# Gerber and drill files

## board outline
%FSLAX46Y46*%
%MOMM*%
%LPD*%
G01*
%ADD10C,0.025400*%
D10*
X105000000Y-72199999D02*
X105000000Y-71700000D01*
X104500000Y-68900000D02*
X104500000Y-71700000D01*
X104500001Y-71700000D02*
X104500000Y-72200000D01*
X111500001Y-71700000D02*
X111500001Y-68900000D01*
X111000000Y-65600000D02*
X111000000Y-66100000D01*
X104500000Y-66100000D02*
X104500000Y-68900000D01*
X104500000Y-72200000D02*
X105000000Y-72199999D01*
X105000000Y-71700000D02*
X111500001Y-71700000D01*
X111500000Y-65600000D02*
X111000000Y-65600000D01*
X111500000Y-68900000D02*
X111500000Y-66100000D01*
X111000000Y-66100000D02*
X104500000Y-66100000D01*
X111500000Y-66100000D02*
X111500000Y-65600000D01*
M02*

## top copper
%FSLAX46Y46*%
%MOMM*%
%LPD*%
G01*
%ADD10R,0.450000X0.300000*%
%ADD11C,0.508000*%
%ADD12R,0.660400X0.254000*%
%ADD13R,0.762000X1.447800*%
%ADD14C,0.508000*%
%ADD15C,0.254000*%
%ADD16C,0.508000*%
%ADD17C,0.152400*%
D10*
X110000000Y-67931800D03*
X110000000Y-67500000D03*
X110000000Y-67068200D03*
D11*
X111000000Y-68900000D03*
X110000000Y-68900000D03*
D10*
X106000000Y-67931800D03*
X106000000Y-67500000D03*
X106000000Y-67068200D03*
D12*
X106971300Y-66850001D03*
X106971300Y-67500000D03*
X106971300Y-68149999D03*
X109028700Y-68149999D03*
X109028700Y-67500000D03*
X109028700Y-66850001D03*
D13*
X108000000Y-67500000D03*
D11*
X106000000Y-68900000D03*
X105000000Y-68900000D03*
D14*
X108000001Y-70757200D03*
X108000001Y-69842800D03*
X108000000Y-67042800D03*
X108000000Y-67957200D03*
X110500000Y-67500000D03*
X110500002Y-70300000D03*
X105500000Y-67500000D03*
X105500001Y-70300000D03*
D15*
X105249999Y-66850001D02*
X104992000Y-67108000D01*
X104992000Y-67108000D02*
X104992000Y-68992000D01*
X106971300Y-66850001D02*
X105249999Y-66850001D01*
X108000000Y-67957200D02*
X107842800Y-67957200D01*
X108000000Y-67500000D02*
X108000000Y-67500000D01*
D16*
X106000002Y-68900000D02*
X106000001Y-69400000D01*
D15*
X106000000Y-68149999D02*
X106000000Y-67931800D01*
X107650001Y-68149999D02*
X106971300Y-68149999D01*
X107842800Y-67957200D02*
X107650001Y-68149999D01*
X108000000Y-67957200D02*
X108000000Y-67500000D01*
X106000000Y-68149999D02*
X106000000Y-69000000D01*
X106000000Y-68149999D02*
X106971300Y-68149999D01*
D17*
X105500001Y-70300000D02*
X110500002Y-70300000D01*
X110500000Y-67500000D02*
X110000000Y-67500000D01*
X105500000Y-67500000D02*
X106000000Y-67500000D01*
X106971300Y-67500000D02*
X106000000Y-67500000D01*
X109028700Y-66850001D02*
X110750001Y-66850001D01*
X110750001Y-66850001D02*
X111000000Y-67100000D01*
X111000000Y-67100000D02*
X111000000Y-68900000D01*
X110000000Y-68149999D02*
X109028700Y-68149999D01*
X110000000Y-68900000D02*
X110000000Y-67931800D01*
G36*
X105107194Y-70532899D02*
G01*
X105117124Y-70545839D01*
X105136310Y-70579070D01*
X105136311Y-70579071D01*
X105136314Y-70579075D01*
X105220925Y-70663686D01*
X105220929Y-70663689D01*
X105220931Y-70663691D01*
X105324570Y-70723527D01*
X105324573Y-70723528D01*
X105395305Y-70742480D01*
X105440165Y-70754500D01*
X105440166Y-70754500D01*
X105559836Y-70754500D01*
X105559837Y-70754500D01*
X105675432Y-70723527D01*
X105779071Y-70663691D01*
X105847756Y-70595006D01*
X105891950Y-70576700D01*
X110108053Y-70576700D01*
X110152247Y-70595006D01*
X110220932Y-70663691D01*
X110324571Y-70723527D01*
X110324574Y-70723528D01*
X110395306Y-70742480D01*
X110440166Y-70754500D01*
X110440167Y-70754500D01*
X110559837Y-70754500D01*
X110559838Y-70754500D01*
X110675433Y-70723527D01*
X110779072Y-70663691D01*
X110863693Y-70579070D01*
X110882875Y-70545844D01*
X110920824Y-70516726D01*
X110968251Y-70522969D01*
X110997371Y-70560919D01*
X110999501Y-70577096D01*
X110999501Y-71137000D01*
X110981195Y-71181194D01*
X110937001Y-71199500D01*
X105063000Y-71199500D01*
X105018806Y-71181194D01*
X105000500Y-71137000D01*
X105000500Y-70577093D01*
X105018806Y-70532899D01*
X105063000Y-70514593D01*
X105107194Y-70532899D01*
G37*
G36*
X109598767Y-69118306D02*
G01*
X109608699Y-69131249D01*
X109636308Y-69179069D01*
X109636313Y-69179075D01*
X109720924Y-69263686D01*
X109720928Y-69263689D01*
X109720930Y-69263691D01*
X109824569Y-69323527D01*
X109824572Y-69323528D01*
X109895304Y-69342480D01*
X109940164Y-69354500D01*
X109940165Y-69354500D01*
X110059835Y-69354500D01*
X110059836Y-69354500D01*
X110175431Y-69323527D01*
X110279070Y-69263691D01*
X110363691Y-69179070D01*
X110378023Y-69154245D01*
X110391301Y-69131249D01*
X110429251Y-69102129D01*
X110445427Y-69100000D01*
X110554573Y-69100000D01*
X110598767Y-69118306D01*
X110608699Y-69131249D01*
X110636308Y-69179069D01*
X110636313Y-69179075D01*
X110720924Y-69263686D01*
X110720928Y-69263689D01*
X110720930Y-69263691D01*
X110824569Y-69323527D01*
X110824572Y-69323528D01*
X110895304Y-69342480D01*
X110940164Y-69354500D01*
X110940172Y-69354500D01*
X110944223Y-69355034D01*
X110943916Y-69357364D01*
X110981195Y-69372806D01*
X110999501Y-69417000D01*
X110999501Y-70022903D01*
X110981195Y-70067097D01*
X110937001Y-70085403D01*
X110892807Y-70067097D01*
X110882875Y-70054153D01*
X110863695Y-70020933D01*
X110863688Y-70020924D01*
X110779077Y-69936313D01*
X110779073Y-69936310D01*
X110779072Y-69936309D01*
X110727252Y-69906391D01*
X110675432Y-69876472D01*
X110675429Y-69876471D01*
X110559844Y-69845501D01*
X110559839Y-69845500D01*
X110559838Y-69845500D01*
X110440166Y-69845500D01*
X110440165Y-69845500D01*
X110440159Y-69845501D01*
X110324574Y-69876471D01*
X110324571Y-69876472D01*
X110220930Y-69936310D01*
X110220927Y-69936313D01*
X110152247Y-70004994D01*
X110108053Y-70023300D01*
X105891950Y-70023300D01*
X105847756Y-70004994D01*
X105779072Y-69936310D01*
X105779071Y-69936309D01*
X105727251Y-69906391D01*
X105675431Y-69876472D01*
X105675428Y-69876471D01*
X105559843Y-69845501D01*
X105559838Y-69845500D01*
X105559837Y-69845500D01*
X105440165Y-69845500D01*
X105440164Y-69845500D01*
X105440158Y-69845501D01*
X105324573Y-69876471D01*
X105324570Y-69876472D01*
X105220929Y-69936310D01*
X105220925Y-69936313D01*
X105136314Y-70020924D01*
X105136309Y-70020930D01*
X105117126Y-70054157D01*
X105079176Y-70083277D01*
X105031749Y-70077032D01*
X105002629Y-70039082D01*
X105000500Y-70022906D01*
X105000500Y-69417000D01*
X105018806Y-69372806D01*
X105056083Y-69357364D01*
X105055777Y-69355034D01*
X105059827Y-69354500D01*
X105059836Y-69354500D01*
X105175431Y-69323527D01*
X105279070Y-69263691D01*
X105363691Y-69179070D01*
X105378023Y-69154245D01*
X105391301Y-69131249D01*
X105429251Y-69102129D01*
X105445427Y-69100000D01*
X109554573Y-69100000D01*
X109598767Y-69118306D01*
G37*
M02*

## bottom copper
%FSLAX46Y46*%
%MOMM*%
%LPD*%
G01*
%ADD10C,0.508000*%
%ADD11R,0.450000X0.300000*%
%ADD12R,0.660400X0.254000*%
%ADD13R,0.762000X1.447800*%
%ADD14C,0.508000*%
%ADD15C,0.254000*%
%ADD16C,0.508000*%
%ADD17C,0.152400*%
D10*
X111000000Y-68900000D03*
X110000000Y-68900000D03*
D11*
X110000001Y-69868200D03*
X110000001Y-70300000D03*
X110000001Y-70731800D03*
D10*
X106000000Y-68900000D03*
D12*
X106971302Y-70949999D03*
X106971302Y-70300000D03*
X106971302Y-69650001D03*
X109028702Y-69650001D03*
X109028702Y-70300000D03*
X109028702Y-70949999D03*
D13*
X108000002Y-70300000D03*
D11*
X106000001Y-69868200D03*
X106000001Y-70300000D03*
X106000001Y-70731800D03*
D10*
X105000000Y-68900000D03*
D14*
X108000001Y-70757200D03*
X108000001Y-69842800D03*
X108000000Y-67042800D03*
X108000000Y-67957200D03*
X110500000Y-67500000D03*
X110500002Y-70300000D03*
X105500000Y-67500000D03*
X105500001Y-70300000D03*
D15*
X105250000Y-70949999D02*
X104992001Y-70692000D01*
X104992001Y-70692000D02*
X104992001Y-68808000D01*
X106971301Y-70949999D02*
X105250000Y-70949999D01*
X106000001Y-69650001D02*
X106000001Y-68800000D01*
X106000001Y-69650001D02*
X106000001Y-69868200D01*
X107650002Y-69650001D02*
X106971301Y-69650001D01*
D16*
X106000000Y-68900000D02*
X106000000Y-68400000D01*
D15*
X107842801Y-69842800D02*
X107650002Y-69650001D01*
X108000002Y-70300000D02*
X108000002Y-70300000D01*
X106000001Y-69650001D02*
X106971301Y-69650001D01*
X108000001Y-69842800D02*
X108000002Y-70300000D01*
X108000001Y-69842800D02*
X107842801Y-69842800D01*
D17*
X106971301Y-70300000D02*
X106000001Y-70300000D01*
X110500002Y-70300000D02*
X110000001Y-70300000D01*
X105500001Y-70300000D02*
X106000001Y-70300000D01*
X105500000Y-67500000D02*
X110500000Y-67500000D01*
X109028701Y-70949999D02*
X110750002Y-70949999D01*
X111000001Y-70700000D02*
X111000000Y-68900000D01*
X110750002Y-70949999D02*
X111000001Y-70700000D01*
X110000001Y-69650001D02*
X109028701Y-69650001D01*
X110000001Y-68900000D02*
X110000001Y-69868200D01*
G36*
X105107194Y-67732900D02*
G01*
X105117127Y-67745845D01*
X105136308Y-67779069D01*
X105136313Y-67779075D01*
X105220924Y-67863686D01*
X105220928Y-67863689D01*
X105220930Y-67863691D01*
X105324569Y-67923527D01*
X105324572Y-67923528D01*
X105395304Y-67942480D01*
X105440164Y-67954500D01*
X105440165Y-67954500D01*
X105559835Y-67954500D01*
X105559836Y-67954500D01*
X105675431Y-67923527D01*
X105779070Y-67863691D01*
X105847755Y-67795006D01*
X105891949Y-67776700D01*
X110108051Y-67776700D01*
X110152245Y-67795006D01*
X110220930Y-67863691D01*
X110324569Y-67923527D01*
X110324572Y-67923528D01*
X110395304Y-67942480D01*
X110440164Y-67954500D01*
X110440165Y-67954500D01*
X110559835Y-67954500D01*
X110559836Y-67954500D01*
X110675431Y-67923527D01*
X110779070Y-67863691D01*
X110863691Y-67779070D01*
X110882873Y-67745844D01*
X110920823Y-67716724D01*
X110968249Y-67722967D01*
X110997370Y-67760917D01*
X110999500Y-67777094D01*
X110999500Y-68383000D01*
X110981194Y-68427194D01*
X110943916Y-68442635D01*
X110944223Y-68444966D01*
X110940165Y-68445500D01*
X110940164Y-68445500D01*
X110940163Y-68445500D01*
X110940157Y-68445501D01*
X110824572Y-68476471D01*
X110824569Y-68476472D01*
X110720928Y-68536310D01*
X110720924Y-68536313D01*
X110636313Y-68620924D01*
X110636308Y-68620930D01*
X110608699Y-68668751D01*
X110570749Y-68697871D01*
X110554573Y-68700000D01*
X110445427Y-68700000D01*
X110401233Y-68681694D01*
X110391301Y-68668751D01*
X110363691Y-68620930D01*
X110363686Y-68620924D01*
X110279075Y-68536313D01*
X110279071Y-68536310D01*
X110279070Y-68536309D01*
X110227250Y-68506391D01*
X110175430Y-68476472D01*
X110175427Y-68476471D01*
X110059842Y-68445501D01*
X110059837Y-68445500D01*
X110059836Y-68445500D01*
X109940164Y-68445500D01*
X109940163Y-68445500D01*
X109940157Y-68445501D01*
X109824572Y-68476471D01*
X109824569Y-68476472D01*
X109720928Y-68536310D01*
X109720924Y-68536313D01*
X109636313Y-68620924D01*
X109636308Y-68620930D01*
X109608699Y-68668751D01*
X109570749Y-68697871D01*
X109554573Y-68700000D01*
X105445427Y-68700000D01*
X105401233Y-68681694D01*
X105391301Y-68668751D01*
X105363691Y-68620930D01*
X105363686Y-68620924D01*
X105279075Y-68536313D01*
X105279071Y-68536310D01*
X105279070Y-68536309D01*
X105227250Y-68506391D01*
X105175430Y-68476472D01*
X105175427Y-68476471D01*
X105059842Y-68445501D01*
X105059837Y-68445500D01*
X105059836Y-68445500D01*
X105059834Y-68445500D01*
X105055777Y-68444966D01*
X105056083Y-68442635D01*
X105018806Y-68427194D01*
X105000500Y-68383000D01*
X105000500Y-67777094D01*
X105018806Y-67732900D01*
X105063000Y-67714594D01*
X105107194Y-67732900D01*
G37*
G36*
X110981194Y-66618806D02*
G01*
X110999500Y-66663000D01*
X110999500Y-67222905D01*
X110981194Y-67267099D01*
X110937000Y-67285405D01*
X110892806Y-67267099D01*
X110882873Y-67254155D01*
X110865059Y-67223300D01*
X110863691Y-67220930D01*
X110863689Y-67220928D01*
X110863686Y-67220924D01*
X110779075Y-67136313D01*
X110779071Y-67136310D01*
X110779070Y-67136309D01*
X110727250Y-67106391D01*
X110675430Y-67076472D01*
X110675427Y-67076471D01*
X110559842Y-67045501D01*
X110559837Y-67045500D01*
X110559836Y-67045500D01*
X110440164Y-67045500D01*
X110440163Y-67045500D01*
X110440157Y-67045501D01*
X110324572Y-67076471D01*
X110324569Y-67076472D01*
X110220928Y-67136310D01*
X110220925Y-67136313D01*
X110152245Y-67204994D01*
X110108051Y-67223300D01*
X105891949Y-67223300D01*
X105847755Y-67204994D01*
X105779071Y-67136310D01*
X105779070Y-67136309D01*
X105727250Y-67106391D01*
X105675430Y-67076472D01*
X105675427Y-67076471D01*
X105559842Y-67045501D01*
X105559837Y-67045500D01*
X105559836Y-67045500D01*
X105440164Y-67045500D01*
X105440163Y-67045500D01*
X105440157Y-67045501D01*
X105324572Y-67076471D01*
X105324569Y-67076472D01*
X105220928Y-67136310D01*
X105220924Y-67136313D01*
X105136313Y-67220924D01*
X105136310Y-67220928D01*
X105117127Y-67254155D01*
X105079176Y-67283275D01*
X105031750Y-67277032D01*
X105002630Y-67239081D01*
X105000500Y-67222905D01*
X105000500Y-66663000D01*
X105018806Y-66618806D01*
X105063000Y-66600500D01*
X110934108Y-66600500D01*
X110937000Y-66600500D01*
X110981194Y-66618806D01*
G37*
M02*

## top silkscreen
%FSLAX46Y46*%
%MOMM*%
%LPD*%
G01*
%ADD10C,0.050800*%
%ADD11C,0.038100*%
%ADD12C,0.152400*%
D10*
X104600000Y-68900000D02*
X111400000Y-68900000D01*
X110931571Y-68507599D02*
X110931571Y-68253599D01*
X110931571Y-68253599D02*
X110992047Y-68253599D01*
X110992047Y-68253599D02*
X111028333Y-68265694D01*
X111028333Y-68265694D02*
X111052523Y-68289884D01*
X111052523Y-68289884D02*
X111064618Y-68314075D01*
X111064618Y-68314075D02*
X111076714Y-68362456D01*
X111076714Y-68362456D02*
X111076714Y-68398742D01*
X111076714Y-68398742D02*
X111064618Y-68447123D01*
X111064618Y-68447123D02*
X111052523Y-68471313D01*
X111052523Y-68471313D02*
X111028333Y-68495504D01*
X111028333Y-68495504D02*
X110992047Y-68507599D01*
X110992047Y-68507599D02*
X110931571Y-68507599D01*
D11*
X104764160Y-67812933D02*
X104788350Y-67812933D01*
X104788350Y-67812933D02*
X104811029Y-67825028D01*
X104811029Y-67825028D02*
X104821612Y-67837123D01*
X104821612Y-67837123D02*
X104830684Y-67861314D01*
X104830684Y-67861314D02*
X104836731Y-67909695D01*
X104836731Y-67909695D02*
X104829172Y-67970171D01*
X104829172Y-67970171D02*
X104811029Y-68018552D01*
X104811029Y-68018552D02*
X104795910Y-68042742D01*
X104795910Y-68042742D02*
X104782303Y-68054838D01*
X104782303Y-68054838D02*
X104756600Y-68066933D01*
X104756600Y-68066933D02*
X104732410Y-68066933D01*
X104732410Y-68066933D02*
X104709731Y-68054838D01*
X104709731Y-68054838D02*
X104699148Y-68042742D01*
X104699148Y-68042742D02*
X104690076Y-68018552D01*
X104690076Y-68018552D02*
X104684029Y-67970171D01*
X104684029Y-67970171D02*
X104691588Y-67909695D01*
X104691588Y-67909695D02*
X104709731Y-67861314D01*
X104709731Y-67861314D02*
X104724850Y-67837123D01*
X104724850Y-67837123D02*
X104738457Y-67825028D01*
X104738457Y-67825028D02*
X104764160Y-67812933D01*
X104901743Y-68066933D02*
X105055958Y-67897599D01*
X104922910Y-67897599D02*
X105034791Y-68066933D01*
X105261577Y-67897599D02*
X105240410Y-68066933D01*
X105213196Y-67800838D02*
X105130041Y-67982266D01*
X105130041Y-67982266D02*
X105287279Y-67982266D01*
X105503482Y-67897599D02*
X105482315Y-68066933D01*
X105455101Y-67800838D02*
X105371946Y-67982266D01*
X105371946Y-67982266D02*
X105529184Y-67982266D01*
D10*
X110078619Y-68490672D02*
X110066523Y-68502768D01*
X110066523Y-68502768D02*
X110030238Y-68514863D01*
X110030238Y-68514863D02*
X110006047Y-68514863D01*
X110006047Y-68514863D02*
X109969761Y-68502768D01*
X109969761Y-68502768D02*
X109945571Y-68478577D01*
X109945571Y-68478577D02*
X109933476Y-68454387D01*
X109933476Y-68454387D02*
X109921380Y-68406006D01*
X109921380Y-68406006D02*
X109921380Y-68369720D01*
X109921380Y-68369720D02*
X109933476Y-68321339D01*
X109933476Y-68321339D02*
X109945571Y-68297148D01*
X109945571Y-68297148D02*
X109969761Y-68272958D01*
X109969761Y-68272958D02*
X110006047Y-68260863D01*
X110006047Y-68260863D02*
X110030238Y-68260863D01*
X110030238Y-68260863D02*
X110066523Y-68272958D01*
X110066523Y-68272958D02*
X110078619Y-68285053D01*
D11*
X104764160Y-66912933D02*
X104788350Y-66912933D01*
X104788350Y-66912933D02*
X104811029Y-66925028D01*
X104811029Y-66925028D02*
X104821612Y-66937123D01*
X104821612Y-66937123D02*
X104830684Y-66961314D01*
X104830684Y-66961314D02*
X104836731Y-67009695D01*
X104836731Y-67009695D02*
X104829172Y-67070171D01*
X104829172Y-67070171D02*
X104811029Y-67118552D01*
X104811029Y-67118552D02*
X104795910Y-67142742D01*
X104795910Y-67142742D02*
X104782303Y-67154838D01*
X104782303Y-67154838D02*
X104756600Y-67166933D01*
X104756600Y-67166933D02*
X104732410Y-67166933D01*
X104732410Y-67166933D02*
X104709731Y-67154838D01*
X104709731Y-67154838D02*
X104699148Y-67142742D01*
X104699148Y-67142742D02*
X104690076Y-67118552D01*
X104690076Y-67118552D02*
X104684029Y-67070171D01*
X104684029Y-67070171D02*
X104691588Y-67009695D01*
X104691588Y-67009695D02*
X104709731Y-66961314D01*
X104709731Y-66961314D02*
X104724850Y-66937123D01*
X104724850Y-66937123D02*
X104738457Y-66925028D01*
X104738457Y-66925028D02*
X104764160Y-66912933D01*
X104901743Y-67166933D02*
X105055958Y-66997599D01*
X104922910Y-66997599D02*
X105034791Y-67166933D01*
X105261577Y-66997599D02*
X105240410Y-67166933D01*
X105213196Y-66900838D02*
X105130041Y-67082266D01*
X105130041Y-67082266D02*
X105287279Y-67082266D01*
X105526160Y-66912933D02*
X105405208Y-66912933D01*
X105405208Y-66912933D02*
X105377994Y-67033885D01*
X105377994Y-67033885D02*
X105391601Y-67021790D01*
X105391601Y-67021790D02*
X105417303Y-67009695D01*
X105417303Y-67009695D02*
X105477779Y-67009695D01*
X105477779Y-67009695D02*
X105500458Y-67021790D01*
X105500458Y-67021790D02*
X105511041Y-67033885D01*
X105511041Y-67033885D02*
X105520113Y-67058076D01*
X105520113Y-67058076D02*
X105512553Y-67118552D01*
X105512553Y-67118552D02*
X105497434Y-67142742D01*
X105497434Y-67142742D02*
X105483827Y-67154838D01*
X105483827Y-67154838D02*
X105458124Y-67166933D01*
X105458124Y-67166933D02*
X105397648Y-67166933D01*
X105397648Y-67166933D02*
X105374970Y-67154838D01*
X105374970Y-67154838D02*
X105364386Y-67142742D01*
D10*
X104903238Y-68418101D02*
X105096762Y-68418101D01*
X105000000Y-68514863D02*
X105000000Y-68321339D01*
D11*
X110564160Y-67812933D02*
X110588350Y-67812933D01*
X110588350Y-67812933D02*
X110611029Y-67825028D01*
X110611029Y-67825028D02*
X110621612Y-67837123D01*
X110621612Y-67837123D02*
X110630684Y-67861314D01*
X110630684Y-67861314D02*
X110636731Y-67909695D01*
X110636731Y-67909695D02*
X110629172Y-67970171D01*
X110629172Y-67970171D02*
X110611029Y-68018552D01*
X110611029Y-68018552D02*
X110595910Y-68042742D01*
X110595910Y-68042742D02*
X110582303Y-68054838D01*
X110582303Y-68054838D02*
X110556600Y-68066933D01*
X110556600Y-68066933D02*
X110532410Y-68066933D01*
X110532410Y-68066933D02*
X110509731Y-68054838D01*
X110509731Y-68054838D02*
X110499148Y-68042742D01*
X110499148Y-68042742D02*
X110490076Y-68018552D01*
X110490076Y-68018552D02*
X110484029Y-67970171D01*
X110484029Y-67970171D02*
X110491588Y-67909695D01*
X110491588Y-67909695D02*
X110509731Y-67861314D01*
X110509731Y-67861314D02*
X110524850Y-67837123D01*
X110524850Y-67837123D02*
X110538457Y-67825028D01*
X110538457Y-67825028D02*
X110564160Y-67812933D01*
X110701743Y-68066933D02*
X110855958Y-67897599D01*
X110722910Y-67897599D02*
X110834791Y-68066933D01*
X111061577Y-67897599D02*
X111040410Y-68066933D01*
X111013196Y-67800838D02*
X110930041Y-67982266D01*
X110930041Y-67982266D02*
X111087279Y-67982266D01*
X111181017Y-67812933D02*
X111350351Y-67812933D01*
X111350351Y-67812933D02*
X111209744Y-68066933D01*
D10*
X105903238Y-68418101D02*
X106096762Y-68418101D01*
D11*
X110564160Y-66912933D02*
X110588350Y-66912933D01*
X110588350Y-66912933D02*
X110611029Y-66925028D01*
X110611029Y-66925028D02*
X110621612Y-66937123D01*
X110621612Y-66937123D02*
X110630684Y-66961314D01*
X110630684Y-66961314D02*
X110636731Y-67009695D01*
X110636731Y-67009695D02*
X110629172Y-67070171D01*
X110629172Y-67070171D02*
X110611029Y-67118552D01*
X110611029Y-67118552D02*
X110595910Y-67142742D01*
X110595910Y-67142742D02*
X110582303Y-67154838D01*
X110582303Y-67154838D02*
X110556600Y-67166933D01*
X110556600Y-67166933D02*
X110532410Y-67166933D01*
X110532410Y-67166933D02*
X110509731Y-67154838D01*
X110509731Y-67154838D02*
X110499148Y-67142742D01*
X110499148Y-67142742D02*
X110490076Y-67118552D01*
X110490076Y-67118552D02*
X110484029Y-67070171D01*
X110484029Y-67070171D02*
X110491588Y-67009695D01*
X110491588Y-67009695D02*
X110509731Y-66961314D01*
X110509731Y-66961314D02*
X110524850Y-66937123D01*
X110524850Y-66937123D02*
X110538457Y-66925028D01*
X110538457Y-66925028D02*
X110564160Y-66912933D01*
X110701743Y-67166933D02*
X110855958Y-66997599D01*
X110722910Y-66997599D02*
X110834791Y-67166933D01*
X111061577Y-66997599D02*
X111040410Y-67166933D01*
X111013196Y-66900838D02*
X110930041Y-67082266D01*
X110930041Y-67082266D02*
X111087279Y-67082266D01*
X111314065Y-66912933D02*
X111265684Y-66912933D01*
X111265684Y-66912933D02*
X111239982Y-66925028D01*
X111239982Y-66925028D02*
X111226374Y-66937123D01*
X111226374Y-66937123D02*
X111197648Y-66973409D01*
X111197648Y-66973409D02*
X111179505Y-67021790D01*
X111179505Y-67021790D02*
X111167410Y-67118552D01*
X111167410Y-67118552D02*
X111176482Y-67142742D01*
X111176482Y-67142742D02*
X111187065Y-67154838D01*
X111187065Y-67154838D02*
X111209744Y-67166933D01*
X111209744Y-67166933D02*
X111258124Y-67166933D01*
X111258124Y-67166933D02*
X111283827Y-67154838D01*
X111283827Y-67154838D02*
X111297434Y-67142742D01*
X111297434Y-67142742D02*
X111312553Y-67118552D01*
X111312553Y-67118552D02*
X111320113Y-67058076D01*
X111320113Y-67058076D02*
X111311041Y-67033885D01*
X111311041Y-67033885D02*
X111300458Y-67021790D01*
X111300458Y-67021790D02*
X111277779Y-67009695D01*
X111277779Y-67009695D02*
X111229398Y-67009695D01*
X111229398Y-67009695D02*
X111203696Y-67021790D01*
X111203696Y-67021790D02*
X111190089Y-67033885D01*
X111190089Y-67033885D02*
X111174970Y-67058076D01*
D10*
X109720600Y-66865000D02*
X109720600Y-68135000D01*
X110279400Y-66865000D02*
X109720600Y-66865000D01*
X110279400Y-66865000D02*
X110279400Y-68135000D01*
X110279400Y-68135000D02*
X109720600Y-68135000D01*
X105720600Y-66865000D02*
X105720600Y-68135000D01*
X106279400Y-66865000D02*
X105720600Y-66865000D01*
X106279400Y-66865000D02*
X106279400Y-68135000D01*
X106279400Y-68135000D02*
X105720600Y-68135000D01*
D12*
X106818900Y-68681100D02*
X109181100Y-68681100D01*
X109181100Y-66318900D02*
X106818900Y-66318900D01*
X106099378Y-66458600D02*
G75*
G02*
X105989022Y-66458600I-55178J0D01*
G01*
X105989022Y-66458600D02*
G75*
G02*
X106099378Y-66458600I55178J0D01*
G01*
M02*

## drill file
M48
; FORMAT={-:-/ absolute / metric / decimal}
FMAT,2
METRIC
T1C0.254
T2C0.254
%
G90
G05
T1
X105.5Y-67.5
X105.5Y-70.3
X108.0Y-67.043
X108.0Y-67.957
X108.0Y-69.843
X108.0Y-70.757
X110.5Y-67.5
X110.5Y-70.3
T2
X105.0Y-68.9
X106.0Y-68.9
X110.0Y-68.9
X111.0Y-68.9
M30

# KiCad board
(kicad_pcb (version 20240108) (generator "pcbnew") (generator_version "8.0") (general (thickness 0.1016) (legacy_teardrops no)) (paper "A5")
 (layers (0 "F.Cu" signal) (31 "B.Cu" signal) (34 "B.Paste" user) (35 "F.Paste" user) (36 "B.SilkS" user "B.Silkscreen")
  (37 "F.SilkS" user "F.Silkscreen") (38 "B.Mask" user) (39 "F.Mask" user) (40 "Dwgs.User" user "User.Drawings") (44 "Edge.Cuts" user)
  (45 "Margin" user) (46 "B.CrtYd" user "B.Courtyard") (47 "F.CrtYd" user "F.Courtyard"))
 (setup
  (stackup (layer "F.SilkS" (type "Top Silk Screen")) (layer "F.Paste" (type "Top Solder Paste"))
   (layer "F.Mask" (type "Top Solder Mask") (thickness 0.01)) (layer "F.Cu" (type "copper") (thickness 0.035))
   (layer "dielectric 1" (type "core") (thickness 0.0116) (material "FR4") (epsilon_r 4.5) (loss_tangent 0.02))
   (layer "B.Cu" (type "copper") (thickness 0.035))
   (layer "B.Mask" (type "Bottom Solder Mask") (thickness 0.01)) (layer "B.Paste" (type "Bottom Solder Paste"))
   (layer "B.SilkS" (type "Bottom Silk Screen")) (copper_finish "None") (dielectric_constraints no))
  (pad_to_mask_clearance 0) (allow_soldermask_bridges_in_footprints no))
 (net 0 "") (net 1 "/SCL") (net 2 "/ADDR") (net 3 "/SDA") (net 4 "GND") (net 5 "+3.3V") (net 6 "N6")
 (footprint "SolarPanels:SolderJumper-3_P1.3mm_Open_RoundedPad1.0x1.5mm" (layer "F.Cu") (at 110 67.5 90)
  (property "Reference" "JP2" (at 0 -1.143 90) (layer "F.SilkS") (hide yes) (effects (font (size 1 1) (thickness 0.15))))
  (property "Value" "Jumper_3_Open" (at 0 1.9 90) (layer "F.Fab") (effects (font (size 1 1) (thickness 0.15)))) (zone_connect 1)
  (fp_line (start 0.635 -0.2794) (end -0.635 -0.2794) (stroke (width 0.0508) (type solid)) (layer "F.SilkS"))
  (fp_line (start 0.635 0.2794) (end 0.635 -0.2794) (stroke (width 0.0508) (type default)) (layer "F.SilkS"))
  (fp_line (start 0.635 0.2794) (end -0.635 0.2794) (stroke (width 0.0508) (type solid)) (layer "F.SilkS"))
  (fp_line (start -0.635 0.2794) (end -0.635 -0.2794) (stroke (width 0.0508) (type default)) (layer "F.SilkS"))
  (pad "1" smd rect (at -0.4318 0 90) (size 0.3 0.45) (layers "F.Cu" "F.Mask") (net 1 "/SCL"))
  (pad "2" smd rect (at 0 0 90) (size 0.3 0.45) (layers "F.Cu" "F.Mask") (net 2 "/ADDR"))
  (pad "3" smd rect (at 0.4318 0 90) (size 0.3 0.45) (layers "F.Cu" "F.Mask") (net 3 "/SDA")))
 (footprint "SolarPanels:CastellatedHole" (layer "F.Cu") (at 111 68.9)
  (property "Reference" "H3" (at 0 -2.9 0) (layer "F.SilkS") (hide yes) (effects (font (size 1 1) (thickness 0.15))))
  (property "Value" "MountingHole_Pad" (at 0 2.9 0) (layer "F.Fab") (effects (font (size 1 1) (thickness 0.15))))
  (pad "1" thru_hole circle (at 0 0) (size 0.508 0.508) (drill 0.254) (layers "*.Cu" "*.Mask") (remove_unused_layers no) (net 3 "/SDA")))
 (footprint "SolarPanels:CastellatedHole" (layer "F.Cu") (at 110 68.9)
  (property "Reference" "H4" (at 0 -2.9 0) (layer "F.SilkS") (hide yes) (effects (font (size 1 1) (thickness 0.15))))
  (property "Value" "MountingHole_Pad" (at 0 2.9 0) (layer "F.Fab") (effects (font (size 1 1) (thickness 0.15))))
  (pad "1" thru_hole circle (at 0 0) (size 0.508 0.508) (drill 0.254) (layers "*.Cu" "*.Mask") (remove_unused_layers no) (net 1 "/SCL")))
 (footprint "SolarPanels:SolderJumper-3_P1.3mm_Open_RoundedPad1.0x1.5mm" (layer "F.Cu") (at 106 67.5 90)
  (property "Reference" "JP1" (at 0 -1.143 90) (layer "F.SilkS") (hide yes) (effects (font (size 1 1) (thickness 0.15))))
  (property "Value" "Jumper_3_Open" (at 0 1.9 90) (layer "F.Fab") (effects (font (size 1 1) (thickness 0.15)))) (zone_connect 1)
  (fp_line (start 0.635 -0.2794) (end -0.635 -0.2794) (stroke (width 0.0508) (type solid)) (layer "F.SilkS"))
  (fp_line (start 0.635 0.2794) (end 0.635 -0.2794) (stroke (width 0.0508) (type default)) (layer "F.SilkS"))
  (fp_line (start 0.635 0.2794) (end -0.635 0.2794) (stroke (width 0.0508) (type solid)) (layer "F.SilkS"))
  (fp_line (start -0.635 0.2794) (end -0.635 -0.2794) (stroke (width 0.0508) (type default)) (layer "F.SilkS"))
  (pad "1" smd rect (at -0.4318 0 90) (size 0.3 0.45) (layers "F.Cu" "F.Mask") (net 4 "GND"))
  (pad "2" smd rect (at 0 0 90) (size 0.3 0.45) (layers "F.Cu" "F.Mask") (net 2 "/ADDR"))
  (pad "3" smd rect (at 0.4318 0 90) (size 0.3 0.45) (layers "F.Cu" "F.Mask") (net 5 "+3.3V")))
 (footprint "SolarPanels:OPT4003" (layer "F.Cu") (at 108 67.5)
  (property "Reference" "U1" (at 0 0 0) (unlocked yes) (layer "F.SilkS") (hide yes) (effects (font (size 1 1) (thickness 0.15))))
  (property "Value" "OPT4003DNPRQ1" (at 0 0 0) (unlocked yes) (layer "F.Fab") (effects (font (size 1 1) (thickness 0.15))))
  (fp_line (start -1.1811 1.1811) (end 1.1811 1.1811) (stroke (width 0.1524) (type solid)) (layer "F.SilkS"))
  (fp_line (start 1.1811 -1.1811) (end -1.1811 -1.1811) (stroke (width 0.1524) (type solid)) (layer "F.SilkS"))
  (fp_circle (center -1.9558 -1.0414) (end -1.9027 -1.0264) (stroke (width 0.1524) (type solid)) (fill none) (layer "F.SilkS"))
  (pad "1" smd rect (at -1.0287 -0.649999) (size 0.6604 0.254) (layers "F.Cu" "F.Paste" "F.Mask") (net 5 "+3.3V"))
  (pad "2" smd rect (at -1.0287 0) (size 0.6604 0.254) (layers "F.Cu" "F.Paste" "F.Mask") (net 2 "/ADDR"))
  (pad "3" smd rect (at -1.0287 0.649999) (size 0.6604 0.254) (layers "F.Cu" "F.Paste" "F.Mask") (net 4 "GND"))
  (pad "4" smd rect (at 1.0287 0.649999) (size 0.6604 0.254) (layers "F.Cu" "F.Paste" "F.Mask") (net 1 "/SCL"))
  (pad "5" smd rect (at 1.0287 0) (size 0.6604 0.254) (layers "F.Cu" "F.Paste" "F.Mask") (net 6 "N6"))
  (pad "6" smd rect (at 1.0287 -0.649999) (size 0.6604 0.254) (layers "F.Cu" "F.Paste" "F.Mask") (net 3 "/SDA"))
  (pad "7" smd rect (at 0 0) (size 0.762 1.4478) (layers "F.Cu" "F.Paste" "F.Mask") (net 4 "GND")))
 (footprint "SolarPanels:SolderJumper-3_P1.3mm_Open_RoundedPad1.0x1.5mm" (layer "B.Cu") (at 110.000001 70.3 -90)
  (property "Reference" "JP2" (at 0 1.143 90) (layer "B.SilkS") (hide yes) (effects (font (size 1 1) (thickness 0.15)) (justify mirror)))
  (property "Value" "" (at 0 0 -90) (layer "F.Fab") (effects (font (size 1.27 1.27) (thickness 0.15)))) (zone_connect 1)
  (pad "1" smd rect (at -0.4318 0 270) (size 0.3 0.45) (layers "B.Cu" "B.Mask") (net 1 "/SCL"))
  (pad "2" smd rect (at 0 0 270) (size 0.3 0.45) (layers "B.Cu" "B.Mask") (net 2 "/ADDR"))
  (pad "3" smd rect (at 0.4318 0 270) (size 0.3 0.45) (layers "B.Cu" "B.Mask") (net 3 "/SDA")))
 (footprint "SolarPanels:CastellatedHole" (layer "B.Cu") (at 106 68.9)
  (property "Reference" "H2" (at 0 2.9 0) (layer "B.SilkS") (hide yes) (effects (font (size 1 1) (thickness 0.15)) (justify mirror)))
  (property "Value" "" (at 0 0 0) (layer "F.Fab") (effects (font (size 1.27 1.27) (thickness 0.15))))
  (pad "1" thru_hole circle (at 0 0) (size 0.508 0.508) (drill 0.254) (layers "*.Cu" "*.Mask") (remove_unused_layers no) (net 4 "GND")))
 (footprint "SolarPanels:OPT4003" (layer "B.Cu") (at 108.000002 70.3)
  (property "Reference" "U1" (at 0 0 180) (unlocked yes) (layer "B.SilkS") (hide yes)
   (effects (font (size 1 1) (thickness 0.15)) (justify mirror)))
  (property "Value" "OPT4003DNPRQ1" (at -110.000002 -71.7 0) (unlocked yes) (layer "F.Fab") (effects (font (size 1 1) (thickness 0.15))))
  (pad "1" smd rect (at -1.0287 0.649999) (size 0.6604 0.254) (layers "B.Cu" "B.Paste" "B.Mask") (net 5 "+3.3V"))
  (pad "2" smd rect (at -1.0287 0) (size 0.6604 0.254) (layers "B.Cu" "B.Paste" "B.Mask") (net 2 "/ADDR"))
  (pad "3" smd rect (at -1.0287 -0.649999) (size 0.6604 0.254) (layers "B.Cu" "B.Paste" "B.Mask") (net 4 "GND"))
  (pad "4" smd rect (at 1.0287 -0.649999) (size 0.6604 0.254) (layers "B.Cu" "B.Paste" "B.Mask") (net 1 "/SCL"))
  (pad "5" smd rect (at 1.0287 0) (size 0.6604 0.254) (layers "B.Cu" "B.Paste" "B.Mask") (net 6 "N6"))
  (pad "6" smd rect (at 1.0287 0.649999) (size 0.6604 0.254) (layers "B.Cu" "B.Paste" "B.Mask") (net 3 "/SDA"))
  (pad "7" smd rect (at 0 0) (size 0.762 1.4478) (layers "B.Cu" "B.Paste" "B.Mask") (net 4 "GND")))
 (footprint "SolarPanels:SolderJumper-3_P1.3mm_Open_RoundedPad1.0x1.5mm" (layer "B.Cu") (at 106.000001 70.3 -90)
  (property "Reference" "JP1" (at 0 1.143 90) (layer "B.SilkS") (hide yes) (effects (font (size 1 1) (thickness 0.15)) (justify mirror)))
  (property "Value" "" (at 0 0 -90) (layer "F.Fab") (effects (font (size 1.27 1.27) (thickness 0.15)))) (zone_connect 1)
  (pad "1" smd rect (at -0.4318 0 270) (size 0.3 0.45) (layers "B.Cu" "B.Mask") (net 4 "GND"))
  (pad "2" smd rect (at 0 0 270) (size 0.3 0.45) (layers "B.Cu" "B.Mask") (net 2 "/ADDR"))
  (pad "3" smd rect (at 0.4318 0 270) (size 0.3 0.45) (layers "B.Cu" "B.Mask") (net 5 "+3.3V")))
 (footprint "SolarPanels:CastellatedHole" (layer "B.Cu") (at 105 68.9)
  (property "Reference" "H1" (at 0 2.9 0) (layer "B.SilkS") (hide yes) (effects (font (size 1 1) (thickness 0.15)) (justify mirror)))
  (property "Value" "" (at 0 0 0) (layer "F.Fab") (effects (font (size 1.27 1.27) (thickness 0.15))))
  (pad "1" thru_hole circle (at 0 0) (size 0.508 0.508) (drill 0.254) (layers "*.Cu" "*.Mask") (remove_unused_layers no) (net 5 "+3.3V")))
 (gr_line (start 104.6 68.9) (end 111.4 68.9) (stroke (width 0.0508) (type default)) (layer "F.SilkS"))
 (gr_line (start 105 72.199999) (end 105 71.7) (stroke (width 0.0254) (type default)) (layer "Edge.Cuts"))
 (gr_line (start 104.5 68.9) (end 104.5 71.7) (stroke (width 0.0254) (type default)) (layer "Edge.Cuts"))
 (gr_line (start 104.500001 71.7) (end 104.5 72.2) (stroke (width 0.0254) (type default)) (layer "Edge.Cuts"))
 (gr_line (start 111.500001 71.7) (end 111.500001 68.9) (stroke (width 0.0254) (type default)) (layer "Edge.Cuts"))
 (gr_line (start 111 65.6) (end 111 66.1) (stroke (width 0.0254) (type default)) (layer "Edge.Cuts"))
 (gr_line (start 104.5 66.1) (end 104.5 68.9) (stroke (width 0.0254) (type default)) (layer "Edge.Cuts"))
 (gr_line (start 104.5 72.2) (end 105 72.199999) (stroke (width 0.0254) (type default)) (layer "Edge.Cuts"))
 (gr_line (start 105 71.7) (end 111.500001 71.7) (stroke (width 0.0254) (type default)) (layer "Edge.Cuts"))
 (gr_line (start 111.5 65.6) (end 111 65.6) (stroke (width 0.0254) (type default)) (layer "Edge.Cuts"))
 (gr_line (start 111.5 68.9) (end 111.5 66.1) (stroke (width 0.0254) (type default)) (layer "Edge.Cuts"))
 (gr_line (start 111 66.1) (end 104.5 66.1) (stroke (width 0.0254) (type default)) (layer "Edge.Cuts"))
 (gr_line (start 111.5 66.1) (end 111.5 65.6) (stroke (width 0.0254) (type default)) (layer "Edge.Cuts"))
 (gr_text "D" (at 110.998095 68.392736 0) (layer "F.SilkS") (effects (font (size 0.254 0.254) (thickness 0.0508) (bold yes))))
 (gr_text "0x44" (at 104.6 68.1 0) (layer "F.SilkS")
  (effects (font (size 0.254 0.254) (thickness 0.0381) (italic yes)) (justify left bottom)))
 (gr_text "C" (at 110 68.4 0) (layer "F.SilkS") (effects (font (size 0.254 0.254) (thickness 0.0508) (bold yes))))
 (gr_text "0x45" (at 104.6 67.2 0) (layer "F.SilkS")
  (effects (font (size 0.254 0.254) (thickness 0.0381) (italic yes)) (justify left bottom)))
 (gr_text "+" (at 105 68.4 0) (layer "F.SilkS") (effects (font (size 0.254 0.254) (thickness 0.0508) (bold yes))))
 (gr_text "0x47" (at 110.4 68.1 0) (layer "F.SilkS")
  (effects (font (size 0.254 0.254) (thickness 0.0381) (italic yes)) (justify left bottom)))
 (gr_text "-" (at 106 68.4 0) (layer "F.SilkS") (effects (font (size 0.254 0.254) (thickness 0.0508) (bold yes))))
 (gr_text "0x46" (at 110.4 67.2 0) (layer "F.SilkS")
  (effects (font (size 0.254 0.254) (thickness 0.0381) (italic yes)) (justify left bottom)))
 (segment (start 105.249999 66.850001) (end 104.992 67.108) (width 0.254) (layer "F.Cu") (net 5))
 (segment (start 104.992 67.108) (end 104.992 68.992) (width 0.254) (layer "F.Cu") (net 5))
 (segment (start 106.9713 66.850001) (end 105.249999 66.850001) (width 0.254) (layer "F.Cu") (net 5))
 (segment (start 105.25 70.949999) (end 104.992001 70.692) (width 0.254) (layer "B.Cu") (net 5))
 (segment (start 104.992001 70.692) (end 104.992001 68.808) (width 0.254) (layer "B.Cu") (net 5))
 (segment (start 106.971301 70.949999) (end 105.25 70.949999) (width 0.254) (layer "B.Cu") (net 5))
 (segment (start 108 67.9572) (end 107.8428 67.9572) (width 0.254) (layer "F.Cu") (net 4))
 (segment (start 108 67.5) (end 108 67.5) (width 0.254) (layer "F.Cu") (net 4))
 (segment (start 106.000002 68.9) (end 106.000001 69.4) (width 0.508) (layer "F.Cu") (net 4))
 (segment (start 106 68.149999) (end 106 67.9318) (width 0.254) (layer "F.Cu") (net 4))
 (segment (start 107.650001 68.149999) (end 106.9713 68.149999) (width 0.254) (layer "F.Cu") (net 4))
 (segment (start 107.8428 67.9572) (end 107.650001 68.149999) (width 0.254) (layer "F.Cu") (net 4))
 (segment (start 108 67.9572) (end 108 67.5) (width 0.254) (layer "F.Cu") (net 4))
 (segment (start 106 68.149999) (end 106 69) (width 0.254) (layer "F.Cu") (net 4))
 (segment (start 106 68.149999) (end 106.9713 68.149999) (width 0.254) (layer "F.Cu") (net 4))
 (via (at 108.000001 70.7572) (size 0.508) (drill 0.254) (layers "F.Cu" "B.Cu") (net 4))
 (via (at 108.000001 69.8428) (size 0.508) (drill 0.254) (layers "F.Cu" "B.Cu") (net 4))
 (via (at 108 67.0428) (size 0.508) (drill 0.254) (layers "F.Cu" "B.Cu") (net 4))
 (via (at 108 67.9572) (size 0.508) (drill 0.254) (layers "F.Cu" "B.Cu") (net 4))
 (segment (start 106.000001 69.650001) (end 106.000001 68.8) (width 0.254) (layer "B.Cu") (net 4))
 (segment (start 106.000001 69.650001) (end 106.000001 69.8682) (width 0.254) (layer "B.Cu") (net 4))
 (segment (start 107.650002 69.650001) (end 106.971301 69.650001) (width 0.254) (layer "B.Cu") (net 4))
 (segment (start 106 68.9) (end 106 68.4) (width 0.508) (layer "B.Cu") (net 4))
 (segment (start 107.842801 69.8428) (end 107.650002 69.650001) (width 0.254) (layer "B.Cu") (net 4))
 (segment (start 108.000002 70.3) (end 108.000002 70.3) (width 0.254) (layer "B.Cu") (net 4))
 (segment (start 106.000001 69.650001) (end 106.971301 69.650001) (width 0.254) (layer "B.Cu") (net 4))
 (segment (start 108.000001 69.8428) (end 108.000002 70.3) (width 0.254) (layer "B.Cu") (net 4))
 (segment (start 108.000001 69.8428) (end 107.842801 69.8428) (width 0.254) (layer "B.Cu") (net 4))
 (segment (start 105.500001 70.3) (end 110.500002 70.3) (width 0.1524) (layer "F.Cu") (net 2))
 (segment (start 110.5 67.5) (end 110 67.5) (width 0.1524) (layer "F.Cu") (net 2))
 (segment (start 105.5 67.5) (end 106 67.5) (width 0.1524) (layer "F.Cu") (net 2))
 (segment (start 106.9713 67.5) (end 106 67.5) (width 0.1524) (layer "F.Cu") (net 2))
 (via (at 110.5 67.5) (size 0.508) (drill 0.254) (layers "F.Cu" "B.Cu") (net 2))
 (via (at 110.500002 70.3) (size 0.508) (drill 0.254) (layers "F.Cu" "B.Cu") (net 2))
 (via (at 105.5 67.5) (size 0.508) (drill 0.254) (layers "F.Cu" "B.Cu") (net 2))
 (via (at 105.500001 70.3) (size 0.508) (drill 0.254) (layers "F.Cu" "B.Cu") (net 2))
 (segment (start 106.971301 70.3) (end 106.000001 70.3) (width 0.1524) (layer "B.Cu") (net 2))
 (segment (start 110.500002 70.3) (end 110.000001 70.3) (width 0.1524) (layer "B.Cu") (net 2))
 (segment (start 105.500001 70.3) (end 106.000001 70.3) (width 0.1524) (layer "B.Cu") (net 2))
 (segment (start 105.5 67.5) (end 110.5 67.5) (width 0.1524) (layer "B.Cu") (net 2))
 (segment (start 109.0287 66.850001) (end 110.750001 66.850001) (width 0.1524) (layer "F.Cu") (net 3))
 (segment (start 110.750001 66.850001) (end 111 67.1) (width 0.1524) (layer "F.Cu") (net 3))
 (segment (start 111 67.1) (end 111 68.9) (width 0.1524) (layer "F.Cu") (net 3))
 (segment (start 109.028701 70.949999) (end 110.750002 70.949999) (width 0.1524) (layer "B.Cu") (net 3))
 (segment (start 111.000001 70.7) (end 111 68.9) (width 0.1524) (layer "B.Cu") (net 3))
 (segment (start 110.750002 70.949999) (end 111.000001 70.7) (width 0.1524) (layer "B.Cu") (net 3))
 (segment (start 110 68.149999) (end 109.0287 68.149999) (width 0.1524) (layer "F.Cu") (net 1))
 (segment (start 110 68.9) (end 110 67.9318) (width 0.1524) (layer "F.Cu") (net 1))
 (segment (start 110.000001 69.650001) (end 109.028701 69.650001) (width 0.1524) (layer "B.Cu") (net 1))
 (segment (start 110.000001 68.9) (end 110.000001 69.8682) (width 0.1524) (layer "B.Cu") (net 1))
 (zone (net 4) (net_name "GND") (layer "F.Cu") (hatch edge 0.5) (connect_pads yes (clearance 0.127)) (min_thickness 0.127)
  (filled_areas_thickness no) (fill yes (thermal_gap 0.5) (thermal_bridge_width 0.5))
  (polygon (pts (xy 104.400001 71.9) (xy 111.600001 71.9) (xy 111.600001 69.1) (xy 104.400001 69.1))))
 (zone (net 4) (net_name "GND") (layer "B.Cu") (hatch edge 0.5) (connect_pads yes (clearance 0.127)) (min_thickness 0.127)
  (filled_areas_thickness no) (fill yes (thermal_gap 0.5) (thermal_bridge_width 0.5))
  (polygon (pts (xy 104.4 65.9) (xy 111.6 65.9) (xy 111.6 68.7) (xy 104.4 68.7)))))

